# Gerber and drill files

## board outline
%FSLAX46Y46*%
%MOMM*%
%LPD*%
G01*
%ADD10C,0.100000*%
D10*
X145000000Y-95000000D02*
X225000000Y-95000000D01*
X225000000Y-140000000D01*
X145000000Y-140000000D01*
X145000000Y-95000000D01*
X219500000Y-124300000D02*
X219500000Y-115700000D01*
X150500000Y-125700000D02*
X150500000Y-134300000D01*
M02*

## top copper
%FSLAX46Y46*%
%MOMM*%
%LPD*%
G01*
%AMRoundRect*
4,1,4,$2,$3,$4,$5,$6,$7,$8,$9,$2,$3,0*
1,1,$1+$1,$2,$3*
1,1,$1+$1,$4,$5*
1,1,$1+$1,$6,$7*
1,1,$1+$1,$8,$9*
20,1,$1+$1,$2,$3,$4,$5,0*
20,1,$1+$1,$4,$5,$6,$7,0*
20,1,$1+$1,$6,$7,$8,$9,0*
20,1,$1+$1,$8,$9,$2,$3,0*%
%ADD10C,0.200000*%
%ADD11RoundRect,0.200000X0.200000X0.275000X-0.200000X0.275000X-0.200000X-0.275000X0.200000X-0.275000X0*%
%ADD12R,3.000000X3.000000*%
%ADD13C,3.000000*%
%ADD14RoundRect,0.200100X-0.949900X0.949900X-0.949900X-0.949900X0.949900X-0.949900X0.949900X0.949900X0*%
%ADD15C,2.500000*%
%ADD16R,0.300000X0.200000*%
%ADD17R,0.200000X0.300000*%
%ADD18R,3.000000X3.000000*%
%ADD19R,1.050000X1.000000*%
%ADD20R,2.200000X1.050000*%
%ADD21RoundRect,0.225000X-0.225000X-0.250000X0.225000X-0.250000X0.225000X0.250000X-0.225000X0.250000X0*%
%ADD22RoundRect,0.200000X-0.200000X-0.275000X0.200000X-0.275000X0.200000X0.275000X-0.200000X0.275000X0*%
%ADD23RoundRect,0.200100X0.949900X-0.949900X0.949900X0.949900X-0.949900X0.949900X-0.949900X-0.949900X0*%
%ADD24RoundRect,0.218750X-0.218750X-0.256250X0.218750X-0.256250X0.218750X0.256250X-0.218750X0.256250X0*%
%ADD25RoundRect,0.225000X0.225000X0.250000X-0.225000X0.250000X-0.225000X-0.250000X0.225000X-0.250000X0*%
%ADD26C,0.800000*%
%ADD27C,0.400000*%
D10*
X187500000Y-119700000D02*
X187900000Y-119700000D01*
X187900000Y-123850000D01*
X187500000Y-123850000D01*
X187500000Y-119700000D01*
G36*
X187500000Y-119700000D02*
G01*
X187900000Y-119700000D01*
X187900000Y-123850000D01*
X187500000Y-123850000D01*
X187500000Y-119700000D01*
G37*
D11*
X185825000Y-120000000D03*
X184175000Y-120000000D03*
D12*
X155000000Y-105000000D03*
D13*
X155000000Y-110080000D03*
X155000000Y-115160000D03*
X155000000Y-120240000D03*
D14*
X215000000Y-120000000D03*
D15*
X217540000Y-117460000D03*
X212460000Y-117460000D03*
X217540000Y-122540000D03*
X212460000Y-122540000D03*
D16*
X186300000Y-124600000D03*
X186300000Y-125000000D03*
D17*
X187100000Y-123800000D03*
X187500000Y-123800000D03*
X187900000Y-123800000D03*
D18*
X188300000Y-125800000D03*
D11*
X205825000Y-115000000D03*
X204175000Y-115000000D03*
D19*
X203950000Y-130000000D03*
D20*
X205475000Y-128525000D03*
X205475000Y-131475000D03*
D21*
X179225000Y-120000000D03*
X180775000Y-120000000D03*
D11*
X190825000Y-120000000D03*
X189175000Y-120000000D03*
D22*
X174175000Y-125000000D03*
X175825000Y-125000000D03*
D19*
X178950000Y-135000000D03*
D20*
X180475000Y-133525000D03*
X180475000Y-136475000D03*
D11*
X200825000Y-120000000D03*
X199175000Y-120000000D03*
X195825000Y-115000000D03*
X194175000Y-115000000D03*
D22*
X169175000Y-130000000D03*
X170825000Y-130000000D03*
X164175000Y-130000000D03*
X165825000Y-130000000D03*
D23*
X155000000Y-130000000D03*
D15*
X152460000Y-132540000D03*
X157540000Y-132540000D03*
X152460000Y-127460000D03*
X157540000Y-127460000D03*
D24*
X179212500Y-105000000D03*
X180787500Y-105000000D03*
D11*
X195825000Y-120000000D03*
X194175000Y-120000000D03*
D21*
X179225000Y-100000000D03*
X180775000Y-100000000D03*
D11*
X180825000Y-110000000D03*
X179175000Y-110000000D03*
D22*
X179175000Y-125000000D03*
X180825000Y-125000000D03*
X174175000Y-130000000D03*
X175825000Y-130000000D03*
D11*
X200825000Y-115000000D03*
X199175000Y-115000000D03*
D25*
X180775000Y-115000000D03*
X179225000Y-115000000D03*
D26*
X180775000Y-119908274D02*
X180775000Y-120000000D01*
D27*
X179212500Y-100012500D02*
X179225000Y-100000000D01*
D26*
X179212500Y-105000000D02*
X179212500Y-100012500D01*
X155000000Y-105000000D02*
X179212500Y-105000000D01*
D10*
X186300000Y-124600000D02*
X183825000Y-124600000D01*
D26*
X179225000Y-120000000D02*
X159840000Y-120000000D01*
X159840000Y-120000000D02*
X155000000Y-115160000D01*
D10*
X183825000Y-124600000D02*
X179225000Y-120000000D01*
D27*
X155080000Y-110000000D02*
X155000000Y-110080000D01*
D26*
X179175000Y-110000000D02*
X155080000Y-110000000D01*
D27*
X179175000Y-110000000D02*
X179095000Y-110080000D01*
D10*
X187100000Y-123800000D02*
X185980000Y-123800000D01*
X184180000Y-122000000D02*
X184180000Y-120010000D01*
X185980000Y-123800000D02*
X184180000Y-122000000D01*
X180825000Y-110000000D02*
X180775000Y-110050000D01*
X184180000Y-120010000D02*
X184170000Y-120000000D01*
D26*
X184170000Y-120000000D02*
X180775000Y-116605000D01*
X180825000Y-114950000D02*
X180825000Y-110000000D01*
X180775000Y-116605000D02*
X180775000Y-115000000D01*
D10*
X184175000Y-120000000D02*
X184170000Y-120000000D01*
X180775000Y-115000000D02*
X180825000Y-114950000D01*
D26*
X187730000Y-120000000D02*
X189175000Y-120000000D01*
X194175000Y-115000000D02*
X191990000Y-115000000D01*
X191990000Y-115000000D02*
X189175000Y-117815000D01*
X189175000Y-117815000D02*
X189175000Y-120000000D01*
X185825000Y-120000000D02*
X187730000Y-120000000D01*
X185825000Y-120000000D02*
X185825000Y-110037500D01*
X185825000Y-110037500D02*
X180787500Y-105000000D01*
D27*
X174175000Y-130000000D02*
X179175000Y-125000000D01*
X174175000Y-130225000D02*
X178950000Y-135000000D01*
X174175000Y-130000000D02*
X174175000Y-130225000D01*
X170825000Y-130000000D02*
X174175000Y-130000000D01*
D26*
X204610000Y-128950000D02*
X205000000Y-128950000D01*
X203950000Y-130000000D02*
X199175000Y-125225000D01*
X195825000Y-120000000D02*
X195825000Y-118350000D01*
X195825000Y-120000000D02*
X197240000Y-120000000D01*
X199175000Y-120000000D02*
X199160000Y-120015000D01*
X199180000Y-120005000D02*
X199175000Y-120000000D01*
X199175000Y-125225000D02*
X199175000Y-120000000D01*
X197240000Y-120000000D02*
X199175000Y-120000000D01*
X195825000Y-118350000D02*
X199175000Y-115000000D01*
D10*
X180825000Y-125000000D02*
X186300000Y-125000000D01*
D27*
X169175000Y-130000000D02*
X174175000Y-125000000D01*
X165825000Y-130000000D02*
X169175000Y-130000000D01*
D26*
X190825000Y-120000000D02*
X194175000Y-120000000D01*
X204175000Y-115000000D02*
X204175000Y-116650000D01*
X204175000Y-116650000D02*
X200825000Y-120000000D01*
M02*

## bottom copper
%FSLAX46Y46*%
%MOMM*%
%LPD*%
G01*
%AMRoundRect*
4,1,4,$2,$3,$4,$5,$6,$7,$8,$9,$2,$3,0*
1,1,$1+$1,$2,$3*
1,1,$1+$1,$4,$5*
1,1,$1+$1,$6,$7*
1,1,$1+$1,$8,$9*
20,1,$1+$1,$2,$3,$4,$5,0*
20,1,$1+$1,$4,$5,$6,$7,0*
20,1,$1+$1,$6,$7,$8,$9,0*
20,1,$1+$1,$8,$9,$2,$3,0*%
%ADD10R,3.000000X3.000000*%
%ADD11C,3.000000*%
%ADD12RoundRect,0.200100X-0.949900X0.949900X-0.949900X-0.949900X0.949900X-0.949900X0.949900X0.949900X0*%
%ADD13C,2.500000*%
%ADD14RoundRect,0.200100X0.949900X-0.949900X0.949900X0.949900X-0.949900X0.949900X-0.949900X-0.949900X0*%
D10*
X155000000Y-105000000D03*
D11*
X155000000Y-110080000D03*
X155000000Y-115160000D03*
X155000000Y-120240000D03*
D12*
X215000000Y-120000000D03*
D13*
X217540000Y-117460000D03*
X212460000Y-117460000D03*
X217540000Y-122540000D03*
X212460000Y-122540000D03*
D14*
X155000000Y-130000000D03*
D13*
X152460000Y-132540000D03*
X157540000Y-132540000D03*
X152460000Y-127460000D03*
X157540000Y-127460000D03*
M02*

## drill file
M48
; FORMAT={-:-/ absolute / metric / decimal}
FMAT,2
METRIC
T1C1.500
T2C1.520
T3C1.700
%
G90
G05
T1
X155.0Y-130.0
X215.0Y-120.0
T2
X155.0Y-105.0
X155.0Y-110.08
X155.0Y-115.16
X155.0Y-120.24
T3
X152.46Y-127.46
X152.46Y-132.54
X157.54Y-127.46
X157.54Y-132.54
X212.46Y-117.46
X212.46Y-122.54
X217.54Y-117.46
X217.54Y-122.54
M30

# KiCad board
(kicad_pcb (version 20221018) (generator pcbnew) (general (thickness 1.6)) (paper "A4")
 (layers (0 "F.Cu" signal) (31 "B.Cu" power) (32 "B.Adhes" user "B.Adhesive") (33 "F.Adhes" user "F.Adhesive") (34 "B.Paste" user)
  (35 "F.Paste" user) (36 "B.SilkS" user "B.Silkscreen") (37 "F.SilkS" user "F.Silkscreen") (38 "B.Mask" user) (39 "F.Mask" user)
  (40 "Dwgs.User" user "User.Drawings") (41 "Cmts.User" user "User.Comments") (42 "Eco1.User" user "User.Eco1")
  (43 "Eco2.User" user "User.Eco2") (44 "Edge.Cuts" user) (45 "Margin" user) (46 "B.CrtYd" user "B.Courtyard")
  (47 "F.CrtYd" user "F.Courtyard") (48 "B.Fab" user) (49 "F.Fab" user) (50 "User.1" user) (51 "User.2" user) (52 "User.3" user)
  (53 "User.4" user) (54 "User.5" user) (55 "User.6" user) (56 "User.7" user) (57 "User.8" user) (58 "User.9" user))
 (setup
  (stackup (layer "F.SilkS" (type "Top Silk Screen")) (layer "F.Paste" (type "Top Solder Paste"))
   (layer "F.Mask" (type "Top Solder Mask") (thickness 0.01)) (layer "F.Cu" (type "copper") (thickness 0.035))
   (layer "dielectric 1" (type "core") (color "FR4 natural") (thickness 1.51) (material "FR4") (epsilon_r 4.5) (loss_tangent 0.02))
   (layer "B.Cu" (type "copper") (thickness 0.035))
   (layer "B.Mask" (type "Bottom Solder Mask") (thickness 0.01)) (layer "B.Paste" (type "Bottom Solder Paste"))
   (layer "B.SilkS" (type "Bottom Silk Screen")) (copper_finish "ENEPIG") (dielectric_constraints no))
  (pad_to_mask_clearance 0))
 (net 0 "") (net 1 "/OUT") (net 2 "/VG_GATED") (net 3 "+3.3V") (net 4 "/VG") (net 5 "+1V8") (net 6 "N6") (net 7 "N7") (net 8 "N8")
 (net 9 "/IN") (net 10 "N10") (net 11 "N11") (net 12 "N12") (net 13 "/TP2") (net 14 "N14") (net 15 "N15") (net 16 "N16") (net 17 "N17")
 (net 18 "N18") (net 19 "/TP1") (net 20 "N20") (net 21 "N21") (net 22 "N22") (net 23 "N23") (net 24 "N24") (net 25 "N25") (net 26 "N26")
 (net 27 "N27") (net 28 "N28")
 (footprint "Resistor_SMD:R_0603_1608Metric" (layer "F.Cu") (at 185 120 180)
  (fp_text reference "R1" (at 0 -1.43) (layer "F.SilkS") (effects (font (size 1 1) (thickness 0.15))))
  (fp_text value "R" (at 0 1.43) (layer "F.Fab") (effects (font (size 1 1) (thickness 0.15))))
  (pad "1" smd roundrect (at -0.825 0 180) (size 0.8 0.95) (layers "F.Cu" "F.Paste" "F.Mask") (roundrect_rratio 0.25) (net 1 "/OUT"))
  (pad "2" smd roundrect (at 0.825 0 180) (size 0.8 0.95) (layers "F.Cu" "F.Paste" "F.Mask") (roundrect_rratio 0.25) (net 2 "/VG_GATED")))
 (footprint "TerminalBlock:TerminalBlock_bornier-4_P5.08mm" (layer "F.Cu") (at 155 105 -90)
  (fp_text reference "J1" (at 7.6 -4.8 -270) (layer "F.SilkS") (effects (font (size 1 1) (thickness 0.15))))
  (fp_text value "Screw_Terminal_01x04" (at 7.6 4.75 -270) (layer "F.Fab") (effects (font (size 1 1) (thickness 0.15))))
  (pad "1" thru_hole rect (at 0 0 270) (size 3 3) (drill 1.52) (layers "*.Cu" "*.Mask") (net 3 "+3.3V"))
  (pad "2" thru_hole circle (at 5.08 0 270) (size 3 3) (drill 1.52) (layers "*.Cu" "*.Mask") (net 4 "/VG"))
  (pad "3" thru_hole circle (at 10.16 0 270) (size 3 3) (drill 1.52) (layers "*.Cu" "*.Mask") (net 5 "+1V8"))
  (pad "4" thru_hole circle (at 15.24 0 270) (size 3 3) (drill 1.52) (layers "*.Cu" "*.Mask") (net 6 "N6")))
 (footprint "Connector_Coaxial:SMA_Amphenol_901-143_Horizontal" (layer "F.Cu") (at 215 120 -90)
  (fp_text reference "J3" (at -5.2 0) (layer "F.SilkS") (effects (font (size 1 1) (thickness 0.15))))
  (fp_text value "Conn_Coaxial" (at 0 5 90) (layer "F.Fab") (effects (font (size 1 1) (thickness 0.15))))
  (fp_line (start 4.3 -4.5) (end -4.3 -4.5) (stroke (width 0.1) (type solid)) (layer "Edge.Cuts"))
  (pad "1" thru_hole roundrect (at 0 0 270) (size 2.3 2.3) (drill 1.5) (layers "*.Cu" "*.Mask") (remove_unused_layers) (keep_end_layers)
   (zone_layer_connections) (roundrect_rratio 0.087) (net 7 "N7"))
  (pad "2" thru_hole circle (at -2.54 -2.54 270) (size 2.5 2.5) (drill 1.7) (layers "*.Cu" "*.Mask") (remove_unused_layers)
   (keep_end_layers) (zone_layer_connections) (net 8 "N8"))
  (pad "2" thru_hole circle (at -2.54 2.54 270) (size 2.5 2.5) (drill 1.7) (layers "*.Cu" "*.Mask") (remove_unused_layers) (keep_end_layers)
   (zone_layer_connections) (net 8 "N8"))
  (pad "2" thru_hole circle (at 2.54 -2.54 270) (size 2.5 2.5) (drill 1.7) (layers "*.Cu" "*.Mask") (remove_unused_layers) (keep_end_layers)
   (zone_layer_connections) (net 8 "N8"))
  (pad "2" thru_hole circle (at 2.54 2.54 270) (size 2.5 2.5) (drill 1.7) (layers "*.Cu" "*.Mask") (remove_unused_layers) (keep_end_layers)
   (zone_layer_connections) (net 8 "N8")))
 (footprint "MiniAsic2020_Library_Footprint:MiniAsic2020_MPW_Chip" (layer "F.Cu") (at 186.8 124.3)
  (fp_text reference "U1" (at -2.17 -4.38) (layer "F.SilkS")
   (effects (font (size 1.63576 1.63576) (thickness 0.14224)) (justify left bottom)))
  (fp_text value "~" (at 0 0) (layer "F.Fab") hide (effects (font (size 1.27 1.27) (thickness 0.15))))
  (pad "1" smd rect (at -0.5 0.3 180) (size 0.3 0.2) (layers "F.Cu" "F.Paste" "F.Mask") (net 5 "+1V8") (die_length 200)
   (thermal_bridge_angle 45))
  (pad "2" smd rect (at -0.5 0.7 180) (size 0.3 0.2) (layers "F.Cu" "F.Paste" "F.Mask") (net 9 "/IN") (thermal_bridge_angle 45))
  (pad "3" smd rect (at 0.3 -0.5 90) (size 0.3 0.2) (layers "F.Cu" "F.Paste" "F.Mask") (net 2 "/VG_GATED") (thermal_bridge_angle 45))
  (pad "4" smd rect (at 0.7 -0.5 90) (size 0.3 0.2) (layers "F.Cu" "F.Paste" "F.Mask") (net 1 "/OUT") (thermal_bridge_angle 45))
  (pad "5" smd rect (at 1.1 -0.5 90) (size 0.3 0.2) (layers "F.Cu" "F.Paste" "F.Mask") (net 1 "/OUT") (thermal_bridge_angle 45))
  (pad "6" smd rect (at 1.5 1.5) (size 3 3) (layers "F.Cu" "F.Paste" "F.Mask") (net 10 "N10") (thermal_bridge_angle 45)))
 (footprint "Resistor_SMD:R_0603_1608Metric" (layer "F.Cu") (at 205 115 180)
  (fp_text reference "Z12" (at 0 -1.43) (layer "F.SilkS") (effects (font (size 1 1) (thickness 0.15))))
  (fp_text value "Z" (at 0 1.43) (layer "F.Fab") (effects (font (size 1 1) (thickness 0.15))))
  (pad "1" smd roundrect (at -0.825 0 180) (size 0.8 0.95) (layers "F.Cu" "F.Paste" "F.Mask") (roundrect_rratio 0.25) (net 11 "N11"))
  (pad "2" smd roundrect (at 0.825 0 180) (size 0.8 0.95) (layers "F.Cu" "F.Paste" "F.Mask") (roundrect_rratio 0.25) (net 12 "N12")))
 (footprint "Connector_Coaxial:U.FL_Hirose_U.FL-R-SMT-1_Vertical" (layer "F.Cu") (at 205 130)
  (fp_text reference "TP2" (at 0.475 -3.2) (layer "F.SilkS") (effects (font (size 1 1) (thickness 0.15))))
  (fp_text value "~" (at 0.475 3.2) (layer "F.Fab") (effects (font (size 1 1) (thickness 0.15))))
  (pad "1" smd rect (at -1.05 0) (size 1.05 1) (layers "F.Cu" "F.Paste" "F.Mask") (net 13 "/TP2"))
  (pad "2" smd rect (at 0.475 -1.475) (size 2.2 1.05) (layers "F.Cu" "F.Paste" "F.Mask") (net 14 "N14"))
  (pad "2" smd rect (at 0.475 1.475) (size 2.2 1.05) (layers "F.Cu" "F.Paste" "F.Mask") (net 14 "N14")))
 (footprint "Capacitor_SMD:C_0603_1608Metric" (layer "F.Cu") (at 180 120)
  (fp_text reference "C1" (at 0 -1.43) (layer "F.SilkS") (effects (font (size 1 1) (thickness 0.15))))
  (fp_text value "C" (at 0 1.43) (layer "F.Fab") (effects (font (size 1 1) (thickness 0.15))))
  (pad "1" smd roundrect (at -0.775 0) (size 0.9 0.95) (layers "F.Cu" "F.Paste" "F.Mask") (roundrect_rratio 0.25) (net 5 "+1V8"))
  (pad "2" smd roundrect (at 0.775 0) (size 0.9 0.95) (layers "F.Cu" "F.Paste" "F.Mask") (roundrect_rratio 0.25) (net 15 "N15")))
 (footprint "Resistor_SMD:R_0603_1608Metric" (layer "F.Cu") (at 190 120 180)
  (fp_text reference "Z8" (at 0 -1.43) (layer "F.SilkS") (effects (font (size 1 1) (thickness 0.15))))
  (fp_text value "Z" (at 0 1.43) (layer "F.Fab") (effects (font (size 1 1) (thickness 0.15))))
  (pad "1" smd roundrect (at -0.825 0 180) (size 0.8 0.95) (layers "F.Cu" "F.Paste" "F.Mask") (roundrect_rratio 0.25) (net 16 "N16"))
  (pad "2" smd roundrect (at 0.825 0 180) (size 0.8 0.95) (layers "F.Cu" "F.Paste" "F.Mask") (roundrect_rratio 0.25) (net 1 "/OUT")))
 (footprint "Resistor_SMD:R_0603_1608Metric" (layer "F.Cu") (at 175 125)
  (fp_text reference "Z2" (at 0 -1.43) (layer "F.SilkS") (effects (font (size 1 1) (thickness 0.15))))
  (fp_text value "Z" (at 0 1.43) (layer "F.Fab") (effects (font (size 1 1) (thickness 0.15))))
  (pad "1" smd roundrect (at -0.825 0) (size 0.8 0.95) (layers "F.Cu" "F.Paste" "F.Mask") (roundrect_rratio 0.25) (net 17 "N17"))
  (pad "2" smd roundrect (at 0.825 0) (size 0.8 0.95) (layers "F.Cu" "F.Paste" "F.Mask") (roundrect_rratio 0.25) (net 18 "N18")))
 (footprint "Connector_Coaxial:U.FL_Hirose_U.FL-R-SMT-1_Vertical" (layer "F.Cu") (at 180 135)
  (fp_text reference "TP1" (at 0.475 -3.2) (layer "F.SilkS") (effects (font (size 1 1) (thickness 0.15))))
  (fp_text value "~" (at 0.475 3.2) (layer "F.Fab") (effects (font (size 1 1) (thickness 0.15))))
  (pad "1" smd rect (at -1.05 0) (size 1.05 1) (layers "F.Cu" "F.Paste" "F.Mask") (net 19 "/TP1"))
  (pad "2" smd rect (at 0.475 -1.475) (size 2.2 1.05) (layers "F.Cu" "F.Paste" "F.Mask") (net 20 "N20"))
  (pad "2" smd rect (at 0.475 1.475) (size 2.2 1.05) (layers "F.Cu" "F.Paste" "F.Mask") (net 20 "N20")))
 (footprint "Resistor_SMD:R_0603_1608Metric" (layer "F.Cu") (at 200 120 180)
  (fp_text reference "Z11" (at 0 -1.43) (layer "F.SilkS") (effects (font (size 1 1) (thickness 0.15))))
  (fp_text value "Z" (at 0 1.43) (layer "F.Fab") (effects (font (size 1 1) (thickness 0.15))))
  (pad "1" smd roundrect (at -0.825 0 180) (size 0.8 0.95) (layers "F.Cu" "F.Paste" "F.Mask") (roundrect_rratio 0.25) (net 12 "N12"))
  (pad "2" smd roundrect (at 0.825 0 180) (size 0.8 0.95) (layers "F.Cu" "F.Paste" "F.Mask") (roundrect_rratio 0.25) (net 13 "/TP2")))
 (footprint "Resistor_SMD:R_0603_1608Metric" (layer "F.Cu") (at 195 115 180)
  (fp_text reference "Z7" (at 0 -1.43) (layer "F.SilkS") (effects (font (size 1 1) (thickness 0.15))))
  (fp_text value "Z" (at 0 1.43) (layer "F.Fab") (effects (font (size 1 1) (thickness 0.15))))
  (pad "1" smd roundrect (at -0.825 0 180) (size 0.8 0.95) (layers "F.Cu" "F.Paste" "F.Mask") (roundrect_rratio 0.25) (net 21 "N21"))
  (pad "2" smd roundrect (at 0.825 0 180) (size 0.8 0.95) (layers "F.Cu" "F.Paste" "F.Mask") (roundrect_rratio 0.25) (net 1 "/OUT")))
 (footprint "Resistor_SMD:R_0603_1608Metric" (layer "F.Cu") (at 170 130)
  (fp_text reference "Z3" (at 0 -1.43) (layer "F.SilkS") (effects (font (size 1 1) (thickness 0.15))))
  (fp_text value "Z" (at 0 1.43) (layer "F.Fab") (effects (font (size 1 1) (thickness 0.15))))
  (pad "1" smd roundrect (at -0.825 0) (size 0.8 0.95) (layers "F.Cu" "F.Paste" "F.Mask") (roundrect_rratio 0.25) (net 17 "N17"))
  (pad "2" smd roundrect (at 0.825 0) (size 0.8 0.95) (layers "F.Cu" "F.Paste" "F.Mask") (roundrect_rratio 0.25) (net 19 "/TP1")))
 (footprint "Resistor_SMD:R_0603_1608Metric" (layer "F.Cu") (at 165 130)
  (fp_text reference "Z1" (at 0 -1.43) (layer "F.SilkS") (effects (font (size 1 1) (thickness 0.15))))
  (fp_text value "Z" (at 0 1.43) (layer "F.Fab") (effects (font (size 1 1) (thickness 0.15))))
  (pad "1" smd roundrect (at -0.825 0) (size 0.8 0.95) (layers "F.Cu" "F.Paste" "F.Mask") (roundrect_rratio 0.25) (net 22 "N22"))
  (pad "2" smd roundrect (at 0.825 0) (size 0.8 0.95) (layers "F.Cu" "F.Paste" "F.Mask") (roundrect_rratio 0.25) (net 17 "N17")))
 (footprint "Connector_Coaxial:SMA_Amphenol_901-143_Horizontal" (layer "F.Cu") (at 155 130 90)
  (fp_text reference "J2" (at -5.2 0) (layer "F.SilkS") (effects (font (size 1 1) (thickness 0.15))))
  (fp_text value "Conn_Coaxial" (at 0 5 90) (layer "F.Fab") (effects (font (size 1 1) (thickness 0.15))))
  (fp_line (start 4.3 -4.5) (end -4.3 -4.5) (stroke (width 0.1) (type solid)) (layer "Edge.Cuts"))
  (pad "1" thru_hole roundrect (at 0 0 90) (size 2.3 2.3) (drill 1.5) (layers "*.Cu" "*.Mask") (remove_unused_layers) (keep_end_layers)
   (zone_layer_connections) (roundrect_rratio 0.087) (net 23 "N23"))
  (pad "2" thru_hole circle (at -2.54 -2.54 90) (size 2.5 2.5) (drill 1.7) (layers "*.Cu" "*.Mask") (remove_unused_layers) (keep_end_layers)
   (zone_layer_connections) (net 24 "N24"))
  (pad "2" thru_hole circle (at -2.54 2.54 90) (size 2.5 2.5) (drill 1.7) (layers "*.Cu" "*.Mask") (remove_unused_layers) (keep_end_layers)
   (zone_layer_connections) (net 24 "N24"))
  (pad "2" thru_hole circle (at 2.54 -2.54 90) (size 2.5 2.5) (drill 1.7) (layers "*.Cu" "*.Mask") (remove_unused_layers) (keep_end_layers)
   (zone_layer_connections) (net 24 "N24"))
  (pad "2" thru_hole circle (at 2.54 2.54 90) (size 2.5 2.5) (drill 1.7) (layers "*.Cu" "*.Mask") (remove_unused_layers) (keep_end_layers)
   (zone_layer_connections) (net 24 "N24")))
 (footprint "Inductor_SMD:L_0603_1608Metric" (layer "F.Cu") (at 180 105)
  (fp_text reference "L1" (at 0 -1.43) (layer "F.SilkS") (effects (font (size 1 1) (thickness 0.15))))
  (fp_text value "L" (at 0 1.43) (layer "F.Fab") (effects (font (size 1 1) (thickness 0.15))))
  (pad "1" smd roundrect (at -0.7875 0) (size 0.875 0.95) (layers "F.Cu" "F.Paste" "F.Mask") (roundrect_rratio 0.25) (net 3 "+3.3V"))
  (pad "2" smd roundrect (at 0.7875 0) (size 0.875 0.95) (layers "F.Cu" "F.Paste" "F.Mask") (roundrect_rratio 0.25) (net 1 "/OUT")))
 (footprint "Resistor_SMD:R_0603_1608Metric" (layer "F.Cu") (at 195 120 180)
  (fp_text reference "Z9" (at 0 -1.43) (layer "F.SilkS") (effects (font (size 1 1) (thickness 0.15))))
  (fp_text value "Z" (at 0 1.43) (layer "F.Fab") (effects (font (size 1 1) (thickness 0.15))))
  (pad "1" smd roundrect (at -0.825 0 180) (size 0.8 0.95) (layers "F.Cu" "F.Paste" "F.Mask") (roundrect_rratio 0.25) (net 13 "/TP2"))
  (pad "2" smd roundrect (at 0.825 0 180) (size 0.8 0.95) (layers "F.Cu" "F.Paste" "F.Mask") (roundrect_rratio 0.25) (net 16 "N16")))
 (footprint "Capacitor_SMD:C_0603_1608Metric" (layer "F.Cu") (at 180 100)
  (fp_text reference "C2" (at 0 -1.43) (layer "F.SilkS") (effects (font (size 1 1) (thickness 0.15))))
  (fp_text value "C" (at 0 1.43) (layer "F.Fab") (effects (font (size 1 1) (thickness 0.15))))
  (pad "1" smd roundrect (at -0.775 0) (size 0.9 0.95) (layers "F.Cu" "F.Paste" "F.Mask") (roundrect_rratio 0.25) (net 3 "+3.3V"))
  (pad "2" smd roundrect (at 0.775 0) (size 0.9 0.95) (layers "F.Cu" "F.Paste" "F.Mask") (roundrect_rratio 0.25) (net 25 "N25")))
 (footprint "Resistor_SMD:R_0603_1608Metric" (layer "F.Cu") (at 180 110 180)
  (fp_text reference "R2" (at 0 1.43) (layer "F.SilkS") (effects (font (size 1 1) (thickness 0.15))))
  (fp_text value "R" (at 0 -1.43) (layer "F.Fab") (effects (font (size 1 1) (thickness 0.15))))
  (pad "1" smd roundrect (at -0.825 0 180) (size 0.8 0.95) (layers "F.Cu" "F.Paste" "F.Mask") (roundrect_rratio 0.25) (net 2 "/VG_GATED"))
  (pad "2" smd roundrect (at 0.825 0 180) (size 0.8 0.95) (layers "F.Cu" "F.Paste" "F.Mask") (roundrect_rratio 0.25) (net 4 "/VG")))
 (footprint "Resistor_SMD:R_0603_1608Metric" (layer "F.Cu") (at 180 125)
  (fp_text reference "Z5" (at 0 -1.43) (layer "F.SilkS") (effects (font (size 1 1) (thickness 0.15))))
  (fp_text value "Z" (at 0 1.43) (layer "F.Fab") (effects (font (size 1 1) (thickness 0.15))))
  (pad "1" smd roundrect (at -0.825 0) (size 0.8 0.95) (layers "F.Cu" "F.Paste" "F.Mask") (roundrect_rratio 0.25) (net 19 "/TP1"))
  (pad "2" smd roundrect (at 0.825 0) (size 0.8 0.95) (layers "F.Cu" "F.Paste" "F.Mask") (roundrect_rratio 0.25) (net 9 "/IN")))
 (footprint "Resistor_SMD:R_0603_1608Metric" (layer "F.Cu") (at 175 130)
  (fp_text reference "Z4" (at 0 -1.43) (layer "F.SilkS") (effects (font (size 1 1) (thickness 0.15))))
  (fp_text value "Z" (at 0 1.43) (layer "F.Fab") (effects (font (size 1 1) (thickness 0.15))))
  (pad "1" smd roundrect (at -0.825 0) (size 0.8 0.95) (layers "F.Cu" "F.Paste" "F.Mask") (roundrect_rratio 0.25) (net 19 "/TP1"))
  (pad "2" smd roundrect (at 0.825 0) (size 0.8 0.95) (layers "F.Cu" "F.Paste" "F.Mask") (roundrect_rratio 0.25) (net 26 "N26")))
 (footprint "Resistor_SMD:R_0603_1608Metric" (layer "F.Cu") (at 200 115 180)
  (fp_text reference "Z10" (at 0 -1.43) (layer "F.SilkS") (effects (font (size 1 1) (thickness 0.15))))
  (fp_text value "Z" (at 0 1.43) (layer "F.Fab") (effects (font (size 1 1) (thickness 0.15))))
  (pad "1" smd roundrect (at -0.825 0 180) (size 0.8 0.95) (layers "F.Cu" "F.Paste" "F.Mask") (roundrect_rratio 0.25) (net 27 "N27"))
  (pad "2" smd roundrect (at 0.825 0 180) (size 0.8 0.95) (layers "F.Cu" "F.Paste" "F.Mask") (roundrect_rratio 0.25) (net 13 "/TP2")))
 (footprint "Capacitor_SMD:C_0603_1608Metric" (layer "F.Cu") (at 180 115 180)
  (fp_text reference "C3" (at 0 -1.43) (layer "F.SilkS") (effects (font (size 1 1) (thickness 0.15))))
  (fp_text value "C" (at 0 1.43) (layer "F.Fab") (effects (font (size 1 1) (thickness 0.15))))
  (pad "1" smd roundrect (at -0.775 0 180) (size 0.9 0.95) (layers "F.Cu" "F.Paste" "F.Mask") (roundrect_rratio 0.25) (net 2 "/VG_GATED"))
  (pad "2" smd roundrect (at 0.775 0 180) (size 0.9 0.95) (layers "F.Cu" "F.Paste" "F.Mask") (roundrect_rratio 0.25) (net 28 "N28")))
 (gr_rect (start 187.5 119.7) (end 187.9 123.85) (stroke (width 0.2) (type solid)) (fill solid) (layer "F.Cu"))
 (gr_rect (start 145 95) (end 225 140) (stroke (width 0.1) (type default)) (fill none) (layer "Edge.Cuts"))
 (segment (start 180.775 119.908274) (end 180.775 120) (width 0.8) (layer "F.Cu") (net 15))
 (segment (start 179.2125 100.0125) (end 179.225 100) (width 0.4) (layer "F.Cu") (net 3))
 (segment (start 179.2125 105) (end 179.2125 100.0125) (width 0.8) (layer "F.Cu") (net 3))
 (segment (start 155 105) (end 179.2125 105) (width 0.8) (layer "F.Cu") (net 3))
 (segment (start 186.3 124.6) (end 183.825 124.6) (width 0.2) (layer "F.Cu") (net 5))
 (segment (start 179.225 120) (end 159.84 120) (width 0.8) (layer "F.Cu") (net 5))
 (segment (start 159.84 120) (end 155 115.16) (width 0.8) (layer "F.Cu") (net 5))
 (segment (start 183.825 124.6) (end 179.225 120) (width 0.2) (layer "F.Cu") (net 5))
 (segment (start 155.08 110) (end 155 110.08) (width 0.4) (layer "F.Cu") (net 4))
 (segment (start 179.175 110) (end 155.08 110) (width 0.8) (layer "F.Cu") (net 4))
 (segment (start 179.175 110) (end 179.095 110.08) (width 0.4) (layer "F.Cu") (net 4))
 (segment (start 187.1 123.8) (end 185.98 123.8) (width 0.2) (layer "F.Cu") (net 2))
 (segment (start 184.18 122) (end 184.18 120.01) (width 0.2) (layer "F.Cu") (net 2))
 (segment (start 185.98 123.8) (end 184.18 122) (width 0.2) (layer "F.Cu") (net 2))
 (segment (start 180.825 110) (end 180.775 110.05) (width 0.2) (layer "F.Cu") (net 2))
 (segment (start 184.18 120.01) (end 184.17 120) (width 0.2) (layer "F.Cu") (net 2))
 (segment (start 184.17 120) (end 180.775 116.605) (width 0.8) (layer "F.Cu") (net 2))
 (segment (start 180.825 114.95) (end 180.825 110) (width 0.8) (layer "F.Cu") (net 2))
 (segment (start 180.775 116.605) (end 180.775 115) (width 0.8) (layer "F.Cu") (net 2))
 (segment (start 184.175 120) (end 184.17 120) (width 0.2) (layer "F.Cu") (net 2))
 (segment (start 180.775 115) (end 180.825 114.95) (width 0.2) (layer "F.Cu") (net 2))
 (segment (start 187.73 120) (end 189.175 120) (width 0.8) (layer "F.Cu") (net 1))
 (segment (start 194.175 115) (end 191.99 115) (width 0.8) (layer "F.Cu") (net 1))
 (segment (start 191.99 115) (end 189.175 117.815) (width 0.8) (layer "F.Cu") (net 1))
 (segment (start 189.175 117.815) (end 189.175 120) (width 0.8) (layer "F.Cu") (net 1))
 (segment (start 185.825 120) (end 187.73 120) (width 0.8) (layer "F.Cu") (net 1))
 (segment (start 185.825 120) (end 185.825 110.0375) (width 0.8) (layer "F.Cu") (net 1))
 (segment (start 185.825 110.0375) (end 180.7875 105) (width 0.8) (layer "F.Cu") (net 1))
 (segment (start 174.175 130) (end 179.175 125) (width 0.4) (layer "F.Cu") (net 19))
 (segment (start 174.175 130.225) (end 178.95 135) (width 0.4) (layer "F.Cu") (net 19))
 (segment (start 174.175 130) (end 174.175 130.225) (width 0.4) (layer "F.Cu") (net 19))
 (segment (start 170.825 130) (end 174.175 130) (width 0.4) (layer "F.Cu") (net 19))
 (segment (start 204.61 128.95) (end 205 128.95) (width 0.8) (layer "F.Cu") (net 14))
 (segment (start 203.95 130) (end 199.175 125.225) (width 0.8) (layer "F.Cu") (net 13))
 (segment (start 195.825 120) (end 195.825 118.35) (width 0.8) (layer "F.Cu") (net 13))
 (segment (start 195.825 120) (end 197.24 120) (width 0.8) (layer "F.Cu") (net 13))
 (segment (start 199.175 120) (end 199.16 120.015) (width 0.8) (layer "F.Cu") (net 13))
 (segment (start 199.18 120.005) (end 199.175 120) (width 0.8) (layer "F.Cu") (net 13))
 (segment (start 199.175 125.225) (end 199.175 120) (width 0.8) (layer "F.Cu") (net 13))
 (segment (start 197.24 120) (end 199.175 120) (width 0.8) (layer "F.Cu") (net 13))
 (segment (start 195.825 118.35) (end 199.175 115) (width 0.8) (layer "F.Cu") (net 13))
 (segment (start 180.825 125) (end 186.3 125) (width 0.2) (layer "F.Cu") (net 9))
 (segment (start 169.175 130) (end 174.175 125) (width 0.4) (layer "F.Cu") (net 17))
 (segment (start 165.825 130) (end 169.175 130) (width 0.4) (layer "F.Cu") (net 17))
 (segment (start 190.825 120) (end 194.175 120) (width 0.8) (layer "F.Cu") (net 16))
 (segment (start 204.175 115) (end 204.175 116.65) (width 0.8) (layer "F.Cu") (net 12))
 (segment (start 204.175 116.65) (end 200.825 120) (width 0.8) (layer "F.Cu") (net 12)))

